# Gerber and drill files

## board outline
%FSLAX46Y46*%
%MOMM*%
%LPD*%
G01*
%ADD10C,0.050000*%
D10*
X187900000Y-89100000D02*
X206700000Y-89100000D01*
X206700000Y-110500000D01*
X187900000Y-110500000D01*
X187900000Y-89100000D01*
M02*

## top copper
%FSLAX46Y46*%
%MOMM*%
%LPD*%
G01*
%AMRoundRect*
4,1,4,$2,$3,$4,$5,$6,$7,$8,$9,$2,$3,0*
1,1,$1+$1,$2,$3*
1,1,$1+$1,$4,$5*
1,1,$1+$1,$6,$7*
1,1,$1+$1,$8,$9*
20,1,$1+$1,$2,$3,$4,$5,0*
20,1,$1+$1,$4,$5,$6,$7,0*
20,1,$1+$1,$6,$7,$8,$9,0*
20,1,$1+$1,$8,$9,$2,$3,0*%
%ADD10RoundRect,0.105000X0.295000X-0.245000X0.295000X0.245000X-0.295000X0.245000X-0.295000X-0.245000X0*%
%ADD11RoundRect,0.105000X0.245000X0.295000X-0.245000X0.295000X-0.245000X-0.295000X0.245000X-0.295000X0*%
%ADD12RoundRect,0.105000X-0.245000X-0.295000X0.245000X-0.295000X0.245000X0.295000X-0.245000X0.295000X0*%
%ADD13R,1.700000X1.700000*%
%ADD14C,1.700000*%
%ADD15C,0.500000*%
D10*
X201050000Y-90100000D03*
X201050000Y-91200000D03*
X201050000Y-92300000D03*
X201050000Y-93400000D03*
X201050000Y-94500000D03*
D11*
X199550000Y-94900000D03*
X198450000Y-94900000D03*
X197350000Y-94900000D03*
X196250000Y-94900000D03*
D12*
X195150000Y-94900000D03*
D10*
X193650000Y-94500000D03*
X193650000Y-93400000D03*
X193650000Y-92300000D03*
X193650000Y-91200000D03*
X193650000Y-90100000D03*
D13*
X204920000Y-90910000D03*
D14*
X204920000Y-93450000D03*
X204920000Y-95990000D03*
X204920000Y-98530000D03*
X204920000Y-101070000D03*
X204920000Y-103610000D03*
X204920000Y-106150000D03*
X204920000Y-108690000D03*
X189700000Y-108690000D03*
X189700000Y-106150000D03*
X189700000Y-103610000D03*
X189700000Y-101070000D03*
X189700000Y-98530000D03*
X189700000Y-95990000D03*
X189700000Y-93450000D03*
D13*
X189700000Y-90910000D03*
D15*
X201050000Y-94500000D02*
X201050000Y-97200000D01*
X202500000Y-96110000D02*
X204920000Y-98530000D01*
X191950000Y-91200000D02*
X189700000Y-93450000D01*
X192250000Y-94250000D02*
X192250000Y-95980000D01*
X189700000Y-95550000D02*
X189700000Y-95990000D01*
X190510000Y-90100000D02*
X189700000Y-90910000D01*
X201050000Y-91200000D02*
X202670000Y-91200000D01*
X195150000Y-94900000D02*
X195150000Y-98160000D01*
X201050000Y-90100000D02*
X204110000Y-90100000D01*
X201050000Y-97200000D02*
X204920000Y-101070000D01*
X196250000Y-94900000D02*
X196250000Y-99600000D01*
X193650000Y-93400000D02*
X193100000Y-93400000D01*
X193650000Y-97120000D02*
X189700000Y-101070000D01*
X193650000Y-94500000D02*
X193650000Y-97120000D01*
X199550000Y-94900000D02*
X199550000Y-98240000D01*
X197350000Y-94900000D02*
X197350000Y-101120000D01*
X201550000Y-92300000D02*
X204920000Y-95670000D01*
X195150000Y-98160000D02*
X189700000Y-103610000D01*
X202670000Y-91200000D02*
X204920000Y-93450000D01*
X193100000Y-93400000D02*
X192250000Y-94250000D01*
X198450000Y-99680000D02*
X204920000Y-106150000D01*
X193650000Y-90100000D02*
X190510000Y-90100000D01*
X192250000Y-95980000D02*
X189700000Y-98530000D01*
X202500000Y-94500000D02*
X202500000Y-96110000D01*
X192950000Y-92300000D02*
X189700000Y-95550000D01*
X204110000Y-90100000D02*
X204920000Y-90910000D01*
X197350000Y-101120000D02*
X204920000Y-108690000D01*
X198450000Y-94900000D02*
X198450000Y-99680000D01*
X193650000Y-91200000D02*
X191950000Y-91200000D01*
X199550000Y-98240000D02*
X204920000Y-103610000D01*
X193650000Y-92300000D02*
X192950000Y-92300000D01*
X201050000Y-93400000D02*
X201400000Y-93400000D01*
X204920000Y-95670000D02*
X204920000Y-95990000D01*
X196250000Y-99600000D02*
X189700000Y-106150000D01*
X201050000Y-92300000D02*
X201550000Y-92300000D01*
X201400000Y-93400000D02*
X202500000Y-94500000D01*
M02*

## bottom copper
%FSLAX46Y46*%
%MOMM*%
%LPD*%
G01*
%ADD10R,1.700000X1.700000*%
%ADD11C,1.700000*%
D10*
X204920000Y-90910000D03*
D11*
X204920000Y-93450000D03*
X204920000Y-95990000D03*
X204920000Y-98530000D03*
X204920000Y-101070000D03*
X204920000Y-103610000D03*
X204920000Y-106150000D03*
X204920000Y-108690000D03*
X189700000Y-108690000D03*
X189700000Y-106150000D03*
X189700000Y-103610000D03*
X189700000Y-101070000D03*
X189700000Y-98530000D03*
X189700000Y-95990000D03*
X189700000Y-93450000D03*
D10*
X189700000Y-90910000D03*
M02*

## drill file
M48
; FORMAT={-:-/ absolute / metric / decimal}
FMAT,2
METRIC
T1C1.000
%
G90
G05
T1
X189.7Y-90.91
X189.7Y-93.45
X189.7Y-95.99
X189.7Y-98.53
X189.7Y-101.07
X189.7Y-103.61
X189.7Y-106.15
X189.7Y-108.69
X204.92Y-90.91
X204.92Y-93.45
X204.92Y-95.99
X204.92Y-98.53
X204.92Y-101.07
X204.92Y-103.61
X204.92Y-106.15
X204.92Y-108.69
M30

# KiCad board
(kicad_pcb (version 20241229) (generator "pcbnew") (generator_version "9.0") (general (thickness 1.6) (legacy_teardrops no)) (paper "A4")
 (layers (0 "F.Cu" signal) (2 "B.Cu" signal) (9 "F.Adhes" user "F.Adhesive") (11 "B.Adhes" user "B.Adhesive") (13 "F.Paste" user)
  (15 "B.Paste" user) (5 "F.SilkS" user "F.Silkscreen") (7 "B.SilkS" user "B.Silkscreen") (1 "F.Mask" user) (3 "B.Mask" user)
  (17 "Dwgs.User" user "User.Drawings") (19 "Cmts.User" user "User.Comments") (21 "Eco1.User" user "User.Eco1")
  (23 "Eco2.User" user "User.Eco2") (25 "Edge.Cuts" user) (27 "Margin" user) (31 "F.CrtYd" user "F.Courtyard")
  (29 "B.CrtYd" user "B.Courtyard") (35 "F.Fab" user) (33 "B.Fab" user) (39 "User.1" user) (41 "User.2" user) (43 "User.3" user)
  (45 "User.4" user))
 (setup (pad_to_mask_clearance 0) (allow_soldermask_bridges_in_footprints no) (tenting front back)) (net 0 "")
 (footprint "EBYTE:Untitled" (layer "F.Cu") (at 196.65 96.6)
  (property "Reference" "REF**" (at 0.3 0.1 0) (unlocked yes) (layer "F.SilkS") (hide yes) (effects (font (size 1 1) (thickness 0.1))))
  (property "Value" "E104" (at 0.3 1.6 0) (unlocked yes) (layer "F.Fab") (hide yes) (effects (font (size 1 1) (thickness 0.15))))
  (pad "1" smd roundrect (at 4.4 -6.5 90) (size 0.7 0.8) (layers "F.Cu" "F.Mask" "F.Paste") (roundrect_rratio 0.15))
  (pad "2" smd roundrect (at 4.4 -5.4 90) (size 0.7 0.8) (layers "F.Cu" "F.Mask" "F.Paste") (roundrect_rratio 0.15))
  (pad "3" smd roundrect (at 4.4 -4.3 90) (size 0.7 0.8) (layers "F.Cu" "F.Mask" "F.Paste") (roundrect_rratio 0.15))
  (pad "4" smd roundrect (at 4.4 -3.2 90) (size 0.7 0.8) (layers "F.Cu" "F.Mask" "F.Paste") (roundrect_rratio 0.15))
  (pad "5" smd roundrect (at 4.4 -2.1 90) (size 0.7 0.8) (layers "F.Cu" "F.Mask" "F.Paste") (roundrect_rratio 0.15))
  (pad "6" smd roundrect (at 2.9 -1.7 180) (size 0.7 0.8) (layers "F.Cu" "F.Mask" "F.Paste") (roundrect_rratio 0.15))
  (pad "7" smd roundrect (at 1.8 -1.7 180) (size 0.7 0.8) (layers "F.Cu" "F.Mask" "F.Paste") (roundrect_rratio 0.15))
  (pad "8" smd roundrect (at 0.7 -1.7 180) (size 0.7 0.8) (layers "F.Cu" "F.Mask" "F.Paste") (roundrect_rratio 0.15))
  (pad "9" smd roundrect (at -0.4 -1.7 180) (size 0.7 0.8) (layers "F.Cu" "F.Mask" "F.Paste") (roundrect_rratio 0.15))
  (pad "10" smd roundrect (at -1.5 -1.7) (size 0.7 0.8) (layers "F.Cu" "F.Mask" "F.Paste") (roundrect_rratio 0.15))
  (pad "11" smd roundrect (at -3 -2.1 90) (size 0.7 0.8) (layers "F.Cu" "F.Mask" "F.Paste") (roundrect_rratio 0.15))
  (pad "12" smd roundrect (at -3 -3.2 90) (size 0.7 0.8) (layers "F.Cu" "F.Mask" "F.Paste") (roundrect_rratio 0.15))
  (pad "13" smd roundrect (at -3 -4.3 90) (size 0.7 0.8) (layers "F.Cu" "F.Mask" "F.Paste") (roundrect_rratio 0.15))
  (pad "14" smd roundrect (at -3 -5.4 90) (size 0.7 0.8) (layers "F.Cu" "F.Mask" "F.Paste") (roundrect_rratio 0.15))
  (pad "15" smd roundrect (at -3 -6.5 90) (size 0.7 0.8) (layers "F.Cu" "F.Mask" "F.Paste") (roundrect_rratio 0.15)))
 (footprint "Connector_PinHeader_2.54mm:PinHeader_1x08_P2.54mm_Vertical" (layer "F.Cu") (at 204.92 90.91)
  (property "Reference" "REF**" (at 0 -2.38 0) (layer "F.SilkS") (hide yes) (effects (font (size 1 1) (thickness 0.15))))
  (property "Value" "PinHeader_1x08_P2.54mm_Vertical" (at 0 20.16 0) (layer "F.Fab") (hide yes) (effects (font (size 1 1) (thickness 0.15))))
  (pad "1" thru_hole rect (at 0 0) (size 1.7 1.7) (drill 1) (layers "*.Cu" "*.Mask") (remove_unused_layers no))
  (pad "2" thru_hole circle (at 0 2.54) (size 1.7 1.7) (drill 1) (layers "*.Cu" "*.Mask") (remove_unused_layers no))
  (pad "3" thru_hole circle (at 0 5.08) (size 1.7 1.7) (drill 1) (layers "*.Cu" "*.Mask") (remove_unused_layers no))
  (pad "4" thru_hole circle (at 0 7.62) (size 1.7 1.7) (drill 1) (layers "*.Cu" "*.Mask") (remove_unused_layers no))
  (pad "5" thru_hole circle (at 0 10.16) (size 1.7 1.7) (drill 1) (layers "*.Cu" "*.Mask") (remove_unused_layers no))
  (pad "6" thru_hole circle (at 0 12.7) (size 1.7 1.7) (drill 1) (layers "*.Cu" "*.Mask") (remove_unused_layers no))
  (pad "7" thru_hole circle (at 0 15.24) (size 1.7 1.7) (drill 1) (layers "*.Cu" "*.Mask") (remove_unused_layers no))
  (pad "8" thru_hole circle (at 0 17.78) (size 1.7 1.7) (drill 1) (layers "*.Cu" "*.Mask") (remove_unused_layers no)))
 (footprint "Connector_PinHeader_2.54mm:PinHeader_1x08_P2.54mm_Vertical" (layer "F.Cu") (at 189.7 90.91)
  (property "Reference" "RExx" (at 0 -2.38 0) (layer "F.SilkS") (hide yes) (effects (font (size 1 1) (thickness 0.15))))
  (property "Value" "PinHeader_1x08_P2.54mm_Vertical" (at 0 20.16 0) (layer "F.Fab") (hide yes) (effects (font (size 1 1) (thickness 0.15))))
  (pad "8" thru_hole circle (at 0 17.78) (size 1.7 1.7) (drill 1) (layers "*.Cu" "*.Mask") (remove_unused_layers no))
  (pad "9" thru_hole circle (at 0 15.24) (size 1.7 1.7) (drill 1) (layers "*.Cu" "*.Mask") (remove_unused_layers no))
  (pad "10" thru_hole circle (at 0 12.7) (size 1.7 1.7) (drill 1) (layers "*.Cu" "*.Mask") (remove_unused_layers no))
  (pad "11" thru_hole circle (at 0 10.16) (size 1.7 1.7) (drill 1) (layers "*.Cu" "*.Mask") (remove_unused_layers no))
  (pad "12" thru_hole circle (at 0 7.62) (size 1.7 1.7) (drill 1) (layers "*.Cu" "*.Mask") (remove_unused_layers no))
  (pad "13" thru_hole circle (at 0 5.08) (size 1.7 1.7) (drill 1) (layers "*.Cu" "*.Mask") (remove_unused_layers no))
  (pad "14" thru_hole circle (at 0 2.54) (size 1.7 1.7) (drill 1) (layers "*.Cu" "*.Mask") (remove_unused_layers no))
  (pad "15" thru_hole rect (at 0 0) (size 1.7 1.7) (drill 1) (layers "*.Cu" "*.Mask") (remove_unused_layers no)))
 (gr_rect (start 187.9 89.1) (end 206.7 110.5) (stroke (width 0.05) (type default)) (fill no) (layer "Edge.Cuts"))
 (segment (start 201.05 94.5) (end 201.05 97.2) (width 0.5) (layer "F.Cu") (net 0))
 (segment (start 202.5 96.11) (end 204.92 98.53) (width 0.5) (layer "F.Cu") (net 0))
 (segment (start 191.95 91.2) (end 189.7 93.45) (width 0.5) (layer "F.Cu") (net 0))
 (segment (start 192.25 94.25) (end 192.25 95.98) (width 0.5) (layer "F.Cu") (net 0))
 (segment (start 189.7 95.55) (end 189.7 95.99) (width 0.5) (layer "F.Cu") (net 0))
 (segment (start 190.51 90.1) (end 189.7 90.91) (width 0.5) (layer "F.Cu") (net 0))
 (segment (start 201.05 91.2) (end 202.67 91.2) (width 0.5) (layer "F.Cu") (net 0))
 (segment (start 195.15 94.9) (end 195.15 98.16) (width 0.5) (layer "F.Cu") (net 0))
 (segment (start 201.05 90.1) (end 204.11 90.1) (width 0.5) (layer "F.Cu") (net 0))
 (segment (start 201.05 97.2) (end 204.92 101.07) (width 0.5) (layer "F.Cu") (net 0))
 (segment (start 196.25 94.9) (end 196.25 99.6) (width 0.5) (layer "F.Cu") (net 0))
 (segment (start 193.65 93.4) (end 193.1 93.4) (width 0.5) (layer "F.Cu") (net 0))
 (segment (start 193.65 97.12) (end 189.7 101.07) (width 0.5) (layer "F.Cu") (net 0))
 (segment (start 193.65 94.5) (end 193.65 97.12) (width 0.5) (layer "F.Cu") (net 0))
 (segment (start 199.55 94.9) (end 199.55 98.24) (width 0.5) (layer "F.Cu") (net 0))
 (segment (start 197.35 94.9) (end 197.35 101.12) (width 0.5) (layer "F.Cu") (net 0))
 (segment (start 201.55 92.3) (end 204.92 95.67) (width 0.5) (layer "F.Cu") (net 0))
 (segment (start 195.15 98.16) (end 189.7 103.61) (width 0.5) (layer "F.Cu") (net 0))
 (segment (start 202.67 91.2) (end 204.92 93.45) (width 0.5) (layer "F.Cu") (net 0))
 (segment (start 193.1 93.4) (end 192.25 94.25) (width 0.5) (layer "F.Cu") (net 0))
 (segment (start 198.45 99.68) (end 204.92 106.15) (width 0.5) (layer "F.Cu") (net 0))
 (segment (start 193.65 90.1) (end 190.51 90.1) (width 0.5) (layer "F.Cu") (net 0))
 (segment (start 192.25 95.98) (end 189.7 98.53) (width 0.5) (layer "F.Cu") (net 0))
 (segment (start 202.5 94.5) (end 202.5 96.11) (width 0.5) (layer "F.Cu") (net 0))
 (segment (start 192.95 92.3) (end 189.7 95.55) (width 0.5) (layer "F.Cu") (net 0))
 (segment (start 204.11 90.1) (end 204.92 90.91) (width 0.5) (layer "F.Cu") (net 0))
 (segment (start 197.35 101.12) (end 204.92 108.69) (width 0.5) (layer "F.Cu") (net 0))
 (segment (start 198.45 94.9) (end 198.45 99.68) (width 0.5) (layer "F.Cu") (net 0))
 (segment (start 193.65 91.2) (end 191.95 91.2) (width 0.5) (layer "F.Cu") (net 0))
 (segment (start 199.55 98.24) (end 204.92 103.61) (width 0.5) (layer "F.Cu") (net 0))
 (segment (start 193.65 92.3) (end 192.95 92.3) (width 0.5) (layer "F.Cu") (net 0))
 (segment (start 201.05 93.4) (end 201.4 93.4) (width 0.5) (layer "F.Cu") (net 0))
 (segment (start 204.92 95.67) (end 204.92 95.99) (width 0.5) (layer "F.Cu") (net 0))
 (segment (start 196.25 99.6) (end 189.7 106.15) (width 0.5) (layer "F.Cu") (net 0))
 (segment (start 201.05 92.3) (end 201.55 92.3) (width 0.5) (layer "F.Cu") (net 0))
 (segment (start 201.4 93.4) (end 202.5 94.5) (width 0.5) (layer "F.Cu") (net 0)))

